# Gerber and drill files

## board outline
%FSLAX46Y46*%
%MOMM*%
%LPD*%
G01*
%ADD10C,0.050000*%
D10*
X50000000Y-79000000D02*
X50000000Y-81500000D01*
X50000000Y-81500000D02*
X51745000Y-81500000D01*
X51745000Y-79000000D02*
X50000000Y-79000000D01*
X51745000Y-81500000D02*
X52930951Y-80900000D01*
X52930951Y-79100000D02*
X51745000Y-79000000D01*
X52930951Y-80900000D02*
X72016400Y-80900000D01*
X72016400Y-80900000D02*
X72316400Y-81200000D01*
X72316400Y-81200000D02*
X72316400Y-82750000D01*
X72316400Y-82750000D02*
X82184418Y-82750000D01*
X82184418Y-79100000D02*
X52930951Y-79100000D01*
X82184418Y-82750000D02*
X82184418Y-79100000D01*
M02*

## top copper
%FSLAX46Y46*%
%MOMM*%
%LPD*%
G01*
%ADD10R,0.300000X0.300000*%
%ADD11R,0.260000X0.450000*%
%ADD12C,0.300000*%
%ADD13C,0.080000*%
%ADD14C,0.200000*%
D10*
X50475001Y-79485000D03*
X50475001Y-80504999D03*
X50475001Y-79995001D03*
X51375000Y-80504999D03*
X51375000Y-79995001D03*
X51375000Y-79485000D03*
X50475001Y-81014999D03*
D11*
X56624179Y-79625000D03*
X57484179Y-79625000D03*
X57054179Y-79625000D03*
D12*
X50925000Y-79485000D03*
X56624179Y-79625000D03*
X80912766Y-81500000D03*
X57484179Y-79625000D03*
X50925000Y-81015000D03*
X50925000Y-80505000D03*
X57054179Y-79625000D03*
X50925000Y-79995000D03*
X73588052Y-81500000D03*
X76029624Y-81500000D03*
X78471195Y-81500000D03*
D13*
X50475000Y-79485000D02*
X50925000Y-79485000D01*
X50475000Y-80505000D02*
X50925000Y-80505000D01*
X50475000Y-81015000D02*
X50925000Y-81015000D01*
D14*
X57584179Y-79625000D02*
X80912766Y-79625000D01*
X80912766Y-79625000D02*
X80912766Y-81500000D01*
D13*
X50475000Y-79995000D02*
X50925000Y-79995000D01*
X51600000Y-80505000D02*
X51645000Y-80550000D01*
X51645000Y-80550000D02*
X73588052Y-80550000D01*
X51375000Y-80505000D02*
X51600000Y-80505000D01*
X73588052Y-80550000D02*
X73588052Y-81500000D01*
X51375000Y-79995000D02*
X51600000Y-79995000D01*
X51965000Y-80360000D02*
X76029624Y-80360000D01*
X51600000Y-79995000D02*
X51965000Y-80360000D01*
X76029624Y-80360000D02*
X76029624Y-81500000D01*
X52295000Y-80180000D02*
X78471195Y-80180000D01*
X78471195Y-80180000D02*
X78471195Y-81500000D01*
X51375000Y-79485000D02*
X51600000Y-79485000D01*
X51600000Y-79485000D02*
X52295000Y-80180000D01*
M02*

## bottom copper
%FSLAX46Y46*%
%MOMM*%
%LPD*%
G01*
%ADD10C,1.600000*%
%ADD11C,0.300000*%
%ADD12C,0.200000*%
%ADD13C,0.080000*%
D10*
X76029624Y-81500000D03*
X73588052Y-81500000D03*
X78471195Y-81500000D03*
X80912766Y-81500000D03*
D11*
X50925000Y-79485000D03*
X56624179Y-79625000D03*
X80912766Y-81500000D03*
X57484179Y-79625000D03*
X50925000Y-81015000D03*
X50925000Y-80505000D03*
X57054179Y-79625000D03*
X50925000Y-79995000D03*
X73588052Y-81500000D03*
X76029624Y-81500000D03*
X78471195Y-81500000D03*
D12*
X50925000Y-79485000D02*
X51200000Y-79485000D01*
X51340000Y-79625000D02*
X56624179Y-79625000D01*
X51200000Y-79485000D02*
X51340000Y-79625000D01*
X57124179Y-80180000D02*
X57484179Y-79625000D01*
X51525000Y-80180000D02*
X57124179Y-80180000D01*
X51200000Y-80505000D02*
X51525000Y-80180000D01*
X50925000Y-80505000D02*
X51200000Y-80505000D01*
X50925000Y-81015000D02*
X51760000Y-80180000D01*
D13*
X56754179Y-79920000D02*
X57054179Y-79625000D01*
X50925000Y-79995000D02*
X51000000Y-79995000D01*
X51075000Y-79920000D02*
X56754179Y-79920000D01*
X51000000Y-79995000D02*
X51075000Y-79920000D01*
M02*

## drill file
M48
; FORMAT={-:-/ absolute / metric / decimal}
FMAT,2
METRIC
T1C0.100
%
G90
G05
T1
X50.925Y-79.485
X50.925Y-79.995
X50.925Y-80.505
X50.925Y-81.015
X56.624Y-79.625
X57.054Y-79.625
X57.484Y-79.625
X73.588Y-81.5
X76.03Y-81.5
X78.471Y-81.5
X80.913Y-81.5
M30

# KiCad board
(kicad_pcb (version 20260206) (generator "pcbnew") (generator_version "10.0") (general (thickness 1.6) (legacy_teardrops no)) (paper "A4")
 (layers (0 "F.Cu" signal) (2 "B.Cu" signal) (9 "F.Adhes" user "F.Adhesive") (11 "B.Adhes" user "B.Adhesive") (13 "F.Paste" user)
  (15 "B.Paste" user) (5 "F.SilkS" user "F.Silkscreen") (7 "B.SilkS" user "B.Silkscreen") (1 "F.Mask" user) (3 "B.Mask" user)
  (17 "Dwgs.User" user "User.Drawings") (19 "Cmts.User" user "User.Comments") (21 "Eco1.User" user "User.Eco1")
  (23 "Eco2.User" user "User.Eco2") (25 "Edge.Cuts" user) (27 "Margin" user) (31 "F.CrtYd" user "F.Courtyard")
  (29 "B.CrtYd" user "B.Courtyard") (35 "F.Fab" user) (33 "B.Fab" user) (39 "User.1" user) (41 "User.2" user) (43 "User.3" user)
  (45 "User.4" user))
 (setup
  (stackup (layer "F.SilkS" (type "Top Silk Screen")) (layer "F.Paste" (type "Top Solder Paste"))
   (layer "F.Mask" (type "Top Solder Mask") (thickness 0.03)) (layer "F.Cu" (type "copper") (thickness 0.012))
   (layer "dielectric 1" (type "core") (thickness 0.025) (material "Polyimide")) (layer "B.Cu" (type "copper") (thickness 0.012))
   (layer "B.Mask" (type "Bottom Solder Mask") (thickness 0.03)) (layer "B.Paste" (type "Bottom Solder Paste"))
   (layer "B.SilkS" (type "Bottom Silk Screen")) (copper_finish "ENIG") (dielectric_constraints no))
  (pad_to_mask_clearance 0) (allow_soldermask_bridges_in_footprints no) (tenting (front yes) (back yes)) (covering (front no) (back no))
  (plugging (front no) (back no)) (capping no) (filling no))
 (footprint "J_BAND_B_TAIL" (layer "F.Cu") (at 50.9 80.25)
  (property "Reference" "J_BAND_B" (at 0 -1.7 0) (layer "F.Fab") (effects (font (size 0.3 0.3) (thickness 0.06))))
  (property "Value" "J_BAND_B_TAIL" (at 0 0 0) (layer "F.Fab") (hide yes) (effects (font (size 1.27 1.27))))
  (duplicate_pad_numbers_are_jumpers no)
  (pad "1" smd rect (at -0.424999 -0.765) (size 0.3 0.3) (layers "F.Cu" "F.Mask") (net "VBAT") (solder_mask_margin 0.05)
   (thermal_bridge_angle 45))
  (pad "2" smd rect (at -0.424999 0.254999) (size 0.3 0.3) (layers "F.Cu" "F.Mask") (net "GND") (solder_mask_margin 0.05)
   (thermal_bridge_angle 45))
  (pad "3" smd rect (at -0.424999 -0.254999) (size 0.3 0.3) (layers "F.Cu" "F.Mask") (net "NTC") (solder_mask_margin 0.05)
   (thermal_bridge_angle 45))
  (pad "4" smd rect (at 0.475 0.254999) (size 0.3 0.3) (layers "F.Cu" "F.Mask") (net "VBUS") (solder_mask_margin 0.05)
   (thermal_bridge_angle 45))
  (pad "5" smd rect (at 0.475 -0.254999) (size 0.3 0.3) (layers "F.Cu" "F.Mask") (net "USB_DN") (solder_mask_margin 0.05)
   (thermal_bridge_angle 45))
  (pad "6" smd rect (at 0.475 -0.765) (size 0.3 0.3) (layers "F.Cu" "F.Mask") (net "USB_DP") (solder_mask_margin 0.05)
   (thermal_bridge_angle 45))
  (pad "7" smd rect (at -0.424999 0.764999) (size 0.3 0.3) (layers "F.Cu" "F.Mask") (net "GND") (solder_mask_margin 0.05)
   (thermal_bridge_angle 45)))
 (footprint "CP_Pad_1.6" (layer "F.Cu") (at 80.912766 81.5)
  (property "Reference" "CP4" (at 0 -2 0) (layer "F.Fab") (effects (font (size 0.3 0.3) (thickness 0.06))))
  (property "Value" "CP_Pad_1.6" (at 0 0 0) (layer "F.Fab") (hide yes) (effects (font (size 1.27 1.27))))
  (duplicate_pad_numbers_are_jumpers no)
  (pad "1" smd circle (at 0 0) (size 1.6 1.6) (layers "B.Cu" "B.Mask") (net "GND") (solder_mask_margin 0.1)))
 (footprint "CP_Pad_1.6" (layer "F.Cu") (at 76.029624 81.5)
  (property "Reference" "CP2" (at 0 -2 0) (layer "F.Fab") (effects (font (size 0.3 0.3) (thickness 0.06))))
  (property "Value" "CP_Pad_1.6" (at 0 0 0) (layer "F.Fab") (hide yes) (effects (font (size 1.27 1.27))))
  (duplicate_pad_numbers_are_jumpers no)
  (pad "1" smd circle (at 0 0) (size 1.6 1.6) (layers "B.Cu" "B.Mask") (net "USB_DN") (solder_mask_margin 0.1)))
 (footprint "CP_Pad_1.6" (layer "F.Cu") (at 78.471195 81.5)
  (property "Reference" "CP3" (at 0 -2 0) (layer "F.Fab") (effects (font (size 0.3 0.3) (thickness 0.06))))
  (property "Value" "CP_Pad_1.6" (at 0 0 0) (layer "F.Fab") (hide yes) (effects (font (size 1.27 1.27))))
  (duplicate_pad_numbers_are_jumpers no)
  (pad "1" smd circle (at 0 0) (size 1.6 1.6) (layers "B.Cu" "B.Mask") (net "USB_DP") (solder_mask_margin 0.1)))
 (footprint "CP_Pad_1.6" (layer "F.Cu") (at 73.588052 81.5)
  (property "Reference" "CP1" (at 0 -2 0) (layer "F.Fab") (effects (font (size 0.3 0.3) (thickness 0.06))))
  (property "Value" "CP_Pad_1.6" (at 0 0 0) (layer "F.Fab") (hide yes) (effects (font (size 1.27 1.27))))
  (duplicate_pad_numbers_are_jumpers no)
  (pad "1" smd circle (at 0 0) (size 1.6 1.6) (layers "B.Cu" "B.Mask") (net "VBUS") (solder_mask_margin 0.1)))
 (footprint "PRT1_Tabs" (layer "F.Cu") (at 57.054179 79.625)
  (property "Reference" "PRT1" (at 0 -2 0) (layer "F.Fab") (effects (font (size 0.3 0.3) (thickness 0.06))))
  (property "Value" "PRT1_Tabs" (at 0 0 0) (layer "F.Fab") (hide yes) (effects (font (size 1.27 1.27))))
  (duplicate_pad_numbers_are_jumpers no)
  (pad "1" smd rect (at -0.43 0) (size 0.26 0.45) (layers "F.Cu" "F.Mask") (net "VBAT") (solder_mask_margin 0.05) (thermal_bridge_angle 45))
  (pad "2" smd rect (at 0.43 0) (size 0.26 0.45) (layers "F.Cu" "F.Mask") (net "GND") (solder_mask_margin 0.05) (thermal_bridge_angle 45))
  (pad "3" smd rect (at 0 0) (size 0.26 0.45) (layers "F.Cu" "F.Mask") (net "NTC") (solder_mask_margin 0.05) (thermal_bridge_angle 45)))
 (gr_line (start 50 79) (end 50 81.5) (stroke (width 0.05) (type default)) (layer "Edge.Cuts"))
 (gr_line (start 50 81.5) (end 51.745 81.5) (stroke (width 0.05) (type default)) (layer "Edge.Cuts"))
 (gr_line (start 51.745 79) (end 50 79) (stroke (width 0.05) (type default)) (layer "Edge.Cuts"))
 (gr_line (start 51.745 81.5) (end 52.930951 80.9) (stroke (width 0.05) (type default)) (layer "Edge.Cuts"))
 (gr_line (start 52.930951 79.1) (end 51.745 79) (stroke (width 0.05) (type default)) (layer "Edge.Cuts"))
 (gr_line (start 52.930951 80.9) (end 72.0164 80.9) (stroke (width 0.05) (type default)) (layer "Edge.Cuts"))
 (gr_line (start 72.0164 80.9) (end 72.3164 81.2) (stroke (width 0.05) (type default)) (layer "Edge.Cuts"))
 (gr_line (start 72.3164 81.2) (end 72.3164 82.75) (stroke (width 0.05) (type default)) (layer "Edge.Cuts"))
 (gr_line (start 72.3164 82.75) (end 82.184418 82.75) (stroke (width 0.05) (type default)) (layer "Edge.Cuts"))
 (gr_line (start 82.184418 79.1) (end 52.930951 79.1) (stroke (width 0.05) (type default)) (layer "Edge.Cuts"))
 (gr_line (start 82.184418 82.75) (end 82.184418 79.1) (stroke (width 0.05) (type default)) (layer "Edge.Cuts"))
 (segment (start 50.475 79.485) (end 50.925 79.485) (width 0.08) (layer "F.Cu") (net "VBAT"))
 (via (at 56.624179 79.625) (size 0.3) (drill 0.1) (layers "F.Cu" "B.Cu") (tenting (front yes) (back yes)) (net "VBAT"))
 (via (at 50.925 79.485) (size 0.3) (drill 0.1) (layers "F.Cu" "B.Cu") (tenting (front yes) (back yes)) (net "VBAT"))
 (segment (start 51.34 79.625) (end 56.624179 79.625) (width 0.2) (layer "B.Cu") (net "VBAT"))
 (segment (start 51.2 79.485) (end 51.34 79.625) (width 0.2) (layer "B.Cu") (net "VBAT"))
 (segment (start 50.925 79.485) (end 51.2 79.485) (width 0.2) (layer "B.Cu") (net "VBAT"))
 (segment (start 50.475 81.015) (end 50.925 81.015) (width 0.08) (layer "F.Cu") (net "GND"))
 (segment (start 50.475 80.505) (end 50.925 80.505) (width 0.08) (layer "F.Cu") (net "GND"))
 (segment (start 80.912766 79.625) (end 80.912766 81.5) (width 0.2) (layer "F.Cu") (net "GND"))
 (segment (start 57.584179 79.625) (end 80.912766 79.625) (width 0.2) (layer "F.Cu") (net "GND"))
 (via (at 50.925 80.505) (size 0.3) (drill 0.1) (layers "F.Cu" "B.Cu") (tenting (front yes) (back yes)) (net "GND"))
 (via (at 57.484179 79.625) (size 0.3) (drill 0.1) (layers "F.Cu" "B.Cu") (tenting (front yes) (back yes)) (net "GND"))
 (via (at 50.925 81.015) (size 0.3) (drill 0.1) (layers "F.Cu" "B.Cu") (tenting (front yes) (back yes)) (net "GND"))
 (via (at 80.912766 81.5) (size 0.3) (drill 0.1) (layers "F.Cu" "B.Cu") (tenting (front yes) (back yes)) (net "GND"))
 (segment (start 50.925 80.505) (end 51.2 80.505) (width 0.2) (layer "B.Cu") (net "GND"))
 (segment (start 51.525 80.18) (end 57.124179 80.18) (width 0.2) (layer "B.Cu") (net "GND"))
 (segment (start 51.2 80.505) (end 51.525 80.18) (width 0.2) (layer "B.Cu") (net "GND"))
 (segment (start 57.124179 80.18) (end 57.484179 79.625) (width 0.2) (layer "B.Cu") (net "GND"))
 (segment (start 50.925 81.015) (end 51.76 80.18) (width 0.2) (layer "B.Cu") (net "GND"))
 (segment (start 50.475 79.995) (end 50.925 79.995) (width 0.08) (layer "F.Cu") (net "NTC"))
 (via (at 50.925 79.995) (size 0.3) (drill 0.1) (layers "F.Cu" "B.Cu") (tenting (front yes) (back yes)) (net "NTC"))
 (via (at 57.054179 79.625) (size 0.3) (drill 0.1) (layers "F.Cu" "B.Cu") (tenting (front yes) (back yes)) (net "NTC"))
 (segment (start 51.075 79.92) (end 56.754179 79.92) (width 0.08) (layer "B.Cu") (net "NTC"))
 (segment (start 51 79.995) (end 51.075 79.92) (width 0.08) (layer "B.Cu") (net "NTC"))
 (segment (start 50.925 79.995) (end 51 79.995) (width 0.08) (layer "B.Cu") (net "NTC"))
 (segment (start 56.754179 79.92) (end 57.054179 79.625) (width 0.08) (layer "B.Cu") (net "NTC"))
 (segment (start 51.6 80.505) (end 51.645 80.55) (width 0.08) (layer "F.Cu") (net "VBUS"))
 (segment (start 73.588052 80.55) (end 73.588052 81.5) (width 0.08) (layer "F.Cu") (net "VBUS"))
 (segment (start 51.645 80.55) (end 73.588052 80.55) (width 0.08) (layer "F.Cu") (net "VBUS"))
 (segment (start 51.375 80.505) (end 51.6 80.505) (width 0.08) (layer "F.Cu") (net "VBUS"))
 (via (at 73.588052 81.5) (size 0.3) (drill 0.1) (layers "F.Cu" "B.Cu") (tenting (front yes) (back yes)) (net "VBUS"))
 (segment (start 51.965 80.36) (end 76.029624 80.36) (width 0.08) (layer "F.Cu") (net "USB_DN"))
 (segment (start 76.029624 80.36) (end 76.029624 81.5) (width 0.08) (layer "F.Cu") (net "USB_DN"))
 (segment (start 51.6 79.995) (end 51.965 80.36) (width 0.08) (layer "F.Cu") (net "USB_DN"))
 (segment (start 51.375 79.995) (end 51.6 79.995) (width 0.08) (layer "F.Cu") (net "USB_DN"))
 (via (at 76.029624 81.5) (size 0.3) (drill 0.1) (layers "F.Cu" "B.Cu") (tenting (front yes) (back yes)) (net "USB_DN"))
 (segment (start 78.471195 80.18) (end 78.471195 81.5) (width 0.08) (layer "F.Cu") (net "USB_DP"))
 (segment (start 52.295 80.18) (end 78.471195 80.18) (width 0.08) (layer "F.Cu") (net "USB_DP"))
 (segment (start 51.375 79.485) (end 51.6 79.485) (width 0.08) (layer "F.Cu") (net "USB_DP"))
 (segment (start 51.6 79.485) (end 52.295 80.18) (width 0.08) (layer "F.Cu") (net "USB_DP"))
 (via (at 78.471195 81.5) (size 0.3) (drill 0.1) (layers "F.Cu" "B.Cu") (tenting (front yes) (back yes)) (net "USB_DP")))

